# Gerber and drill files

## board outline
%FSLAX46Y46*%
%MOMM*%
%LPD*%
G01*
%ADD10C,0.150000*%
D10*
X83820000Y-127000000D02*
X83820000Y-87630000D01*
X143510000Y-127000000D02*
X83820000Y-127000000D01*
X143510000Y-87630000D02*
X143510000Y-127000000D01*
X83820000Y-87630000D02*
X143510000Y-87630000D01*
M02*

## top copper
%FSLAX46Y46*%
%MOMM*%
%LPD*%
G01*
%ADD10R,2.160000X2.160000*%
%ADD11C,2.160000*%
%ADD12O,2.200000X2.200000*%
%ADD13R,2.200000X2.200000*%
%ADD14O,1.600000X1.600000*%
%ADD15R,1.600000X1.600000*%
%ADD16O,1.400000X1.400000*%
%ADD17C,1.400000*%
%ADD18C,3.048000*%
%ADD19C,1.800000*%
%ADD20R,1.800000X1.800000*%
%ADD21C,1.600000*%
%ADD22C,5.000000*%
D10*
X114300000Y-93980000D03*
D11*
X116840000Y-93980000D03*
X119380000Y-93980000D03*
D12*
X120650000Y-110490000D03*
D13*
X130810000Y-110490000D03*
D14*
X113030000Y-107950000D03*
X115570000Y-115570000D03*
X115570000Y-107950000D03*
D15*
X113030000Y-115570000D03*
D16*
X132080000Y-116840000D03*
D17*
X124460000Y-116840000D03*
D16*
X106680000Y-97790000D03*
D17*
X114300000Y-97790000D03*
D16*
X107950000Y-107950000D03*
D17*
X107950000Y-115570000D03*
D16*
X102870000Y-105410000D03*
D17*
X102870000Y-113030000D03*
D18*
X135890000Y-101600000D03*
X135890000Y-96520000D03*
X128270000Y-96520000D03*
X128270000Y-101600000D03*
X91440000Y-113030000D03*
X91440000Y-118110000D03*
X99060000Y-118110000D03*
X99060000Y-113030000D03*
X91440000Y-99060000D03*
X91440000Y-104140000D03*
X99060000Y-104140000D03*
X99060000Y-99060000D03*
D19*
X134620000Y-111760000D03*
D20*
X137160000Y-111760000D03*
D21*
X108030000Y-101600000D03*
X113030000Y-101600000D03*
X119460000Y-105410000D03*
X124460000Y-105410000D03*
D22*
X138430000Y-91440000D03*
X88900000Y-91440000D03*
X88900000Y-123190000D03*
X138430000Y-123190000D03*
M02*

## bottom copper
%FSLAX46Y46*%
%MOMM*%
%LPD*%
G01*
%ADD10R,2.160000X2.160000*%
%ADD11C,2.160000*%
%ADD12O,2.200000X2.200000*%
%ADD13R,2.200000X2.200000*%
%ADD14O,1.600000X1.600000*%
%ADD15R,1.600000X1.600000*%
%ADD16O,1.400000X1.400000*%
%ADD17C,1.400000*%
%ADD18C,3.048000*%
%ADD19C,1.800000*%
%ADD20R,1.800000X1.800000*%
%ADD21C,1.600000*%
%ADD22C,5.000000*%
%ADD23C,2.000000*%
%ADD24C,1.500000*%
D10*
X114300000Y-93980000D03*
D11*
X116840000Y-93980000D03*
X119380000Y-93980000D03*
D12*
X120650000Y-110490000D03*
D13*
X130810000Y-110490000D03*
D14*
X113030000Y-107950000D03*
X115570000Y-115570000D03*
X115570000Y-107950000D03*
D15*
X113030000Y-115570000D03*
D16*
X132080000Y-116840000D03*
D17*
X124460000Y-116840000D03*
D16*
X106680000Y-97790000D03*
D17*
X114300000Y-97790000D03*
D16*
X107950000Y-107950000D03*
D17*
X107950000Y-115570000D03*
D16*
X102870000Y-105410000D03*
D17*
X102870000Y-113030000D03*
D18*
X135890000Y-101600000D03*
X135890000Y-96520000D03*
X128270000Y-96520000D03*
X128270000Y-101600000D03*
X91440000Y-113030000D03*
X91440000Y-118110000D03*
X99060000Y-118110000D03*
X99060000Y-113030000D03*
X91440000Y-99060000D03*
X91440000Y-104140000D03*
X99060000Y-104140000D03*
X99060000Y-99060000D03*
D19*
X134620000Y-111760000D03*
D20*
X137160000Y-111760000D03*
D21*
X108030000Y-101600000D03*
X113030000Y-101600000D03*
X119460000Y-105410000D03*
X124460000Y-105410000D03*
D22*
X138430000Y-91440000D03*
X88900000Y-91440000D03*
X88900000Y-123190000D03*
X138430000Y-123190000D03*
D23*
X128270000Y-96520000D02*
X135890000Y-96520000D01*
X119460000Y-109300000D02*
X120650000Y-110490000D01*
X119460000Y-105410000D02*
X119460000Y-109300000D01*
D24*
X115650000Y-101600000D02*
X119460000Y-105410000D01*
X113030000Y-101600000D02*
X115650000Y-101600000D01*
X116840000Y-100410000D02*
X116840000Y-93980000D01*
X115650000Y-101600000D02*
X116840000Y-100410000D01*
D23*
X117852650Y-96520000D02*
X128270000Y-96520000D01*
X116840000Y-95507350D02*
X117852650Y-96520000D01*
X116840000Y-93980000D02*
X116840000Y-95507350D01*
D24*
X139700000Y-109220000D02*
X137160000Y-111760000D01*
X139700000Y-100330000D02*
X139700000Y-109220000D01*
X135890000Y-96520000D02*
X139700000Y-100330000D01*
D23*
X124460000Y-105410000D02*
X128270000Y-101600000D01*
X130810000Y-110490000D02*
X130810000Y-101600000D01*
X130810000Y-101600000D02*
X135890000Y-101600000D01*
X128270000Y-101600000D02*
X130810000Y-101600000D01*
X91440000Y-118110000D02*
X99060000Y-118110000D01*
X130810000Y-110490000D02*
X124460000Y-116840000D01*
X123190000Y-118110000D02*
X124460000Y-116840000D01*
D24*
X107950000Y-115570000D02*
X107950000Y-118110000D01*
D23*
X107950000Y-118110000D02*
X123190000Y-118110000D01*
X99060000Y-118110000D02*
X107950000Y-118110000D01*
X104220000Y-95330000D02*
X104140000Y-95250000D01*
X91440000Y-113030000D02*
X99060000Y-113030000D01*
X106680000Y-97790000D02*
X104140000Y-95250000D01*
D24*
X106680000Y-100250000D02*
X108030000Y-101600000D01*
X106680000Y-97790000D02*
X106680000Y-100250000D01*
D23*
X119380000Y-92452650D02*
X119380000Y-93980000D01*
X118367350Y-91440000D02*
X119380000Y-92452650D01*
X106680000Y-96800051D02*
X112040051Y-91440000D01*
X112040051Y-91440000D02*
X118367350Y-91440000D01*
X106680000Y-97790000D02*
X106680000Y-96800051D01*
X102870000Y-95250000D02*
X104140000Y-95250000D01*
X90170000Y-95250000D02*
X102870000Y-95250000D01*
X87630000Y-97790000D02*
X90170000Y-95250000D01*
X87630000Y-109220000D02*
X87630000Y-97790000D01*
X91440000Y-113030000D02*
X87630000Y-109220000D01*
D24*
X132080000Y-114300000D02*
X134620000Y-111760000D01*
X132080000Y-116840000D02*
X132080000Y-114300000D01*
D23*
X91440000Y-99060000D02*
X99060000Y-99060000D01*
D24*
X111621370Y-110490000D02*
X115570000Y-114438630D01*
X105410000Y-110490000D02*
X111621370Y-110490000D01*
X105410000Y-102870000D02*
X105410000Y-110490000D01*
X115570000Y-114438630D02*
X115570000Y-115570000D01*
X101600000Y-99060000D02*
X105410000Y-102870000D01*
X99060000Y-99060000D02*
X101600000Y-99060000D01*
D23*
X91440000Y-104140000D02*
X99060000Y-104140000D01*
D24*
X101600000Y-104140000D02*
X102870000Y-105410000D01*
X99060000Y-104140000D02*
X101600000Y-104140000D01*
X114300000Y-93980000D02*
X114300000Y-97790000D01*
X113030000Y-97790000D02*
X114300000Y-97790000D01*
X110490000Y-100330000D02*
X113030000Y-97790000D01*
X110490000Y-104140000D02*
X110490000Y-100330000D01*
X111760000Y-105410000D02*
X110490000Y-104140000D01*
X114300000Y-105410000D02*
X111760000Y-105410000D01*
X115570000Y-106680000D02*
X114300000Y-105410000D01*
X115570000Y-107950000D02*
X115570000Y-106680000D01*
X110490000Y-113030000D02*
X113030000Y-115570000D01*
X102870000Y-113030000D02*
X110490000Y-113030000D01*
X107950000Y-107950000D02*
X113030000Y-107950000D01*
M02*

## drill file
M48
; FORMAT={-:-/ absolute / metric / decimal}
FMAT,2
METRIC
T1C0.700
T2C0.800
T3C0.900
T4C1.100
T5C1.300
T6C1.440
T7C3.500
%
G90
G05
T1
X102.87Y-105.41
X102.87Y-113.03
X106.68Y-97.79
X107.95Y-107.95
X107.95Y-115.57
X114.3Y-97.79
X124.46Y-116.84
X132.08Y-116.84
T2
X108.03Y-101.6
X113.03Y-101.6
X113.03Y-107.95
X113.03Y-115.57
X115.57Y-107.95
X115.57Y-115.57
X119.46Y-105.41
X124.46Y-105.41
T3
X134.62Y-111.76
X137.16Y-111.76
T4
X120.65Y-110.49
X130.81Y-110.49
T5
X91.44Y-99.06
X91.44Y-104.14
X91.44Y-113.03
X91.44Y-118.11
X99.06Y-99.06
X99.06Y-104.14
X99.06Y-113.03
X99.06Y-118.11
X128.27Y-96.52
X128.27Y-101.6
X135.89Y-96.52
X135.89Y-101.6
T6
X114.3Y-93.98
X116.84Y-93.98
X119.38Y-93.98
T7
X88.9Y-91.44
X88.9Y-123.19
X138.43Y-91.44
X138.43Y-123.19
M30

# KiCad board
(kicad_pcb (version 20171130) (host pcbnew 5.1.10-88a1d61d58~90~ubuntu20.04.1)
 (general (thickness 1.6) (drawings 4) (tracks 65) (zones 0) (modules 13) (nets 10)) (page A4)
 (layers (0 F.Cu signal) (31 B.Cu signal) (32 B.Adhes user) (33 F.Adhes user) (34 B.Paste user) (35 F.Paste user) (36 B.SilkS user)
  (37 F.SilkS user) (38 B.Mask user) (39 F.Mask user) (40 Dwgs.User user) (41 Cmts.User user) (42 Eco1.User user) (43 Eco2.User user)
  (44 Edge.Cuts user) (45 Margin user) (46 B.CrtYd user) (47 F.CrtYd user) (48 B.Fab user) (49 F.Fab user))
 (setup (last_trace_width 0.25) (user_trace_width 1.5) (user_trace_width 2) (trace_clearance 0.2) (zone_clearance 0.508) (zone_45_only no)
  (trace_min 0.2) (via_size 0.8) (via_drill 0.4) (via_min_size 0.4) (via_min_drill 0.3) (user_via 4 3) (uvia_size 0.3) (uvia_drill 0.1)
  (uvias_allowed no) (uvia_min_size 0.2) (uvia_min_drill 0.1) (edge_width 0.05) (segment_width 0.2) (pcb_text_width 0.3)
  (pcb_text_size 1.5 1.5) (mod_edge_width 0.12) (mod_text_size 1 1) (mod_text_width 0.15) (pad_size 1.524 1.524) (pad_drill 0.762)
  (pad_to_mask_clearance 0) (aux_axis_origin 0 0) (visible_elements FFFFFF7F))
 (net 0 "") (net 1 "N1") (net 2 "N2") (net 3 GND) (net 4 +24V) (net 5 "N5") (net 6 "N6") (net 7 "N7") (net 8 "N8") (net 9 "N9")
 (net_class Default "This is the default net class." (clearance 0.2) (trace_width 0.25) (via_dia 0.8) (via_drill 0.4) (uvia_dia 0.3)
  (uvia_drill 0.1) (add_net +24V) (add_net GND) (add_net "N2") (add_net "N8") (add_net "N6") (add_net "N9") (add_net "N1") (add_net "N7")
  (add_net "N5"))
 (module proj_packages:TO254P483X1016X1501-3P (layer F.Cu) (at 114.3 93.98)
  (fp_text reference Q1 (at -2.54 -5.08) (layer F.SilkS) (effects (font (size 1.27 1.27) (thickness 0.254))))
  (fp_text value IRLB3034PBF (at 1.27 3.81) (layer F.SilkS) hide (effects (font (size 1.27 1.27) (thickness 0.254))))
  (pad 1 thru_hole rect (at 0 0) (size 2.16 2.16) (drill 1.44) (layers *.Cu *.Mask) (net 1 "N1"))
  (pad 2 thru_hole circle (at 2.54 0) (size 2.16 2.16) (drill 1.44) (layers *.Cu *.Mask) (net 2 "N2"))
  (pad 3 thru_hole circle (at 5.08 0) (size 2.16 2.16) (drill 1.44) (layers *.Cu *.Mask) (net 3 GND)))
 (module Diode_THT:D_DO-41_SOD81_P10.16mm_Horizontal (layer F.Cu) (at 130.81 110.49 180)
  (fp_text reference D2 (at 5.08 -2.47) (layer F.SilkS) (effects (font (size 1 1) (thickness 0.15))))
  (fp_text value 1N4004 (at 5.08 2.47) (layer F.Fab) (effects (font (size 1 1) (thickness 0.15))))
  (pad 2 thru_hole oval (at 10.16 0 180) (size 2.2 2.2) (drill 1.1) (layers *.Cu *.Mask) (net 2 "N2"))
  (pad 1 thru_hole rect (at 0 0 180) (size 2.2 2.2) (drill 1.1) (layers *.Cu *.Mask) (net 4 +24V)))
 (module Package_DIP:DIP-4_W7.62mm (layer F.Cu) (at 113.03 115.57 90)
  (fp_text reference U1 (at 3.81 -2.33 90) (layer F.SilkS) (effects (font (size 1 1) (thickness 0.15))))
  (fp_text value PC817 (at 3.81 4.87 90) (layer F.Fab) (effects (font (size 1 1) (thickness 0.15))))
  (pad 4 thru_hole oval (at 7.62 0 90) (size 1.6 1.6) (drill 0.8) (layers *.Cu *.Mask) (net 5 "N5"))
  (pad 2 thru_hole oval (at 0 2.54 90) (size 1.6 1.6) (drill 0.8) (layers *.Cu *.Mask) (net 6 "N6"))
  (pad 3 thru_hole oval (at 7.62 2.54 90) (size 1.6 1.6) (drill 0.8) (layers *.Cu *.Mask) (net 1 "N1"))
  (pad 1 thru_hole rect (at 0 0 90) (size 1.6 1.6) (drill 0.8) (layers *.Cu *.Mask) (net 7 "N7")))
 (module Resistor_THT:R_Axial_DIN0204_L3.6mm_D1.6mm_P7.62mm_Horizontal (layer F.Cu) (at 124.46 116.84)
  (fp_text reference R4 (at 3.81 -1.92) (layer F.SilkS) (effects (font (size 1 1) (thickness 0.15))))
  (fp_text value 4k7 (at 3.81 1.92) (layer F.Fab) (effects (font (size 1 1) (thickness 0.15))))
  (pad 2 thru_hole oval (at 7.62 0) (size 1.4 1.4) (drill 0.7) (layers *.Cu *.Mask) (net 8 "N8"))
  (pad 1 thru_hole circle (at 0 0) (size 1.4 1.4) (drill 0.7) (layers *.Cu *.Mask) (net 4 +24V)))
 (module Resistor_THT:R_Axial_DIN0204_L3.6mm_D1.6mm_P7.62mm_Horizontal (layer F.Cu) (at 114.3 97.79 180)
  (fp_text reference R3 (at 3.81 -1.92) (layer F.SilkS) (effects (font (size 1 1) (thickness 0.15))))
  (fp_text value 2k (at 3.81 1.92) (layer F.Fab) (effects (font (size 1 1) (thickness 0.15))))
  (pad 2 thru_hole oval (at 7.62 0 180) (size 1.4 1.4) (drill 0.7) (layers *.Cu *.Mask) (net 3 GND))
  (pad 1 thru_hole circle (at 0 0 180) (size 1.4 1.4) (drill 0.7) (layers *.Cu *.Mask) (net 1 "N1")))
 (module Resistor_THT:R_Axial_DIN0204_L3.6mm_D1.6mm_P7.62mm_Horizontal (layer F.Cu) (at 107.95 115.57 90)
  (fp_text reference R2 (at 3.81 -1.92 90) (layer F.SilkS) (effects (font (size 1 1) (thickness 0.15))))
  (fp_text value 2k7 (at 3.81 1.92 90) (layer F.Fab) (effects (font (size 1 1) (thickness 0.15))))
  (pad 2 thru_hole oval (at 7.62 0 90) (size 1.4 1.4) (drill 0.7) (layers *.Cu *.Mask) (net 5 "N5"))
  (pad 1 thru_hole circle (at 0 0 90) (size 1.4 1.4) (drill 0.7) (layers *.Cu *.Mask) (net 4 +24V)))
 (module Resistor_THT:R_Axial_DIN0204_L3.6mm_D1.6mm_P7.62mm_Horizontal (layer F.Cu) (at 102.87 113.03 90)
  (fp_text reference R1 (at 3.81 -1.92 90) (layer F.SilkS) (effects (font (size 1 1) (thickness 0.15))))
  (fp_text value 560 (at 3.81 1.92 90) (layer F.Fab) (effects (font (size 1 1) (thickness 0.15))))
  (pad 2 thru_hole oval (at 7.62 0 90) (size 1.4 1.4) (drill 0.7) (layers *.Cu *.Mask) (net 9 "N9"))
  (pad 1 thru_hole circle (at 0 0 90) (size 1.4 1.4) (drill 0.7) (layers *.Cu *.Mask) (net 7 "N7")))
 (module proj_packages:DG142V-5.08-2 (layer F.Cu) (at 135.89 99.06 90)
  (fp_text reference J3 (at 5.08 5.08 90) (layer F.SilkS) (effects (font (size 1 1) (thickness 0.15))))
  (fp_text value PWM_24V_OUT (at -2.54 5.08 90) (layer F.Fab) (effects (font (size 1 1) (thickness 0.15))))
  (pad 1 thru_hole circle (at -2.54 0 90) (size 3.048 3.048) (drill 1.3) (layers *.Cu *.Mask) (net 4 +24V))
  (pad 2 thru_hole circle (at 2.54 0 90) (size 3.048 3.048) (drill 1.3) (layers *.Cu *.Mask) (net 2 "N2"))
  (pad 2 thru_hole circle (at 2.54 -7.62 90) (size 3.048 3.048) (drill 1.3) (layers *.Cu *.Mask) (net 2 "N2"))
  (pad 1 thru_hole circle (at -2.54 -7.62 90) (size 3.048 3.048) (drill 1.3) (layers *.Cu *.Mask) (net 4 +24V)))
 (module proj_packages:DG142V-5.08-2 (layer F.Cu) (at 91.44 115.57 270)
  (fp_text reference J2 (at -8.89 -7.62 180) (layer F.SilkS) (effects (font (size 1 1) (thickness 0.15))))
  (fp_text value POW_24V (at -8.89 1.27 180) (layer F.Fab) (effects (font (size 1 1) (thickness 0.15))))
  (pad 1 thru_hole circle (at -2.54 0 270) (size 3.048 3.048) (drill 1.3) (layers *.Cu *.Mask) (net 3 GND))
  (pad 2 thru_hole circle (at 2.54 0 270) (size 3.048 3.048) (drill 1.3) (layers *.Cu *.Mask) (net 4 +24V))
  (pad 2 thru_hole circle (at 2.54 -7.62 270) (size 3.048 3.048) (drill 1.3) (layers *.Cu *.Mask) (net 4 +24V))
  (pad 1 thru_hole circle (at -2.54 -7.62 270) (size 3.048 3.048) (drill 1.3) (layers *.Cu *.Mask) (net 3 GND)))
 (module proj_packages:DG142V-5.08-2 (layer F.Cu) (at 91.44 101.6 270)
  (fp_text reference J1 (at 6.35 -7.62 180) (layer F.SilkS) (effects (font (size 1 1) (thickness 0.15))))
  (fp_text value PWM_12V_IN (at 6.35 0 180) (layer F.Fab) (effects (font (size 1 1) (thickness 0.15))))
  (pad 1 thru_hole circle (at -2.54 0 270) (size 3.048 3.048) (drill 1.3) (layers *.Cu *.Mask) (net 6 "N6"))
  (pad 2 thru_hole circle (at 2.54 0 270) (size 3.048 3.048) (drill 1.3) (layers *.Cu *.Mask) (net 9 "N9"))
  (pad 2 thru_hole circle (at 2.54 -7.62 270) (size 3.048 3.048) (drill 1.3) (layers *.Cu *.Mask) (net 9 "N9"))
  (pad 1 thru_hole circle (at -2.54 -7.62 270) (size 3.048 3.048) (drill 1.3) (layers *.Cu *.Mask) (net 6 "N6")))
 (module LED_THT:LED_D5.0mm (layer F.Cu) (at 137.16 111.76 180)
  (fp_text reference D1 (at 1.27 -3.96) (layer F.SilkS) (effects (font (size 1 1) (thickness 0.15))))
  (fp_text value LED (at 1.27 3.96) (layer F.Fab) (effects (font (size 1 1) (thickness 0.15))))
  (pad 2 thru_hole circle (at 2.54 0 180) (size 1.8 1.8) (drill 0.9) (layers *.Cu *.Mask) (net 8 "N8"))
  (pad 1 thru_hole rect (at 0 0 180) (size 1.8 1.8) (drill 0.9) (layers *.Cu *.Mask) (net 2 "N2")))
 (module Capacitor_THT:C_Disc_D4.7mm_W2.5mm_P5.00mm (layer F.Cu) (at 113.03 101.6 180)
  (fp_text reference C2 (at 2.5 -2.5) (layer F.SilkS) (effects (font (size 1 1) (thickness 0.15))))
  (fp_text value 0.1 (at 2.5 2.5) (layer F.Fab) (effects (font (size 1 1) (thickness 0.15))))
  (pad 2 thru_hole circle (at 5 0 180) (size 1.6 1.6) (drill 0.8) (layers *.Cu *.Mask) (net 3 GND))
  (pad 1 thru_hole circle (at 0 0 180) (size 1.6 1.6) (drill 0.8) (layers *.Cu *.Mask) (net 2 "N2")))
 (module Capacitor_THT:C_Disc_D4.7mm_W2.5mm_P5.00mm (layer F.Cu) (at 124.46 105.41 180)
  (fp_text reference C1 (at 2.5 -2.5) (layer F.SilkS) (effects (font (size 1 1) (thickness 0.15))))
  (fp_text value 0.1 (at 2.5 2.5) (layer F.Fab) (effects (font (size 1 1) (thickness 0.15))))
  (pad 2 thru_hole circle (at 5 0 180) (size 1.6 1.6) (drill 0.8) (layers *.Cu *.Mask) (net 2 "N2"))
  (pad 1 thru_hole circle (at 0 0 180) (size 1.6 1.6) (drill 0.8) (layers *.Cu *.Mask) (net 4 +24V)))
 (gr_line (start 83.82 127) (end 83.82 87.63) (layer Edge.Cuts) (width 0.15))
 (gr_line (start 143.51 127) (end 83.82 127) (layer Edge.Cuts) (width 0.15))
 (gr_line (start 143.51 87.63) (end 143.51 127) (layer Edge.Cuts) (width 0.15))
 (gr_line (start 83.82 87.63) (end 143.51 87.63) (layer Edge.Cuts) (width 0.15))
 (via (at 138.43 91.44) (size 5) (drill 3.5) (layers F.Cu B.Cu) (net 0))
 (via (at 88.9 91.44) (size 5) (drill 3.5) (layers F.Cu B.Cu) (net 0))
 (via (at 88.9 123.19) (size 5) (drill 3.5) (layers F.Cu B.Cu) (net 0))
 (via (at 138.43 123.19) (size 5) (drill 3.5) (layers F.Cu B.Cu) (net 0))
 (segment (start 128.27 96.52) (end 135.89 96.52) (width 2) (layer B.Cu) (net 2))
 (segment (start 119.46 109.3) (end 120.65 110.49) (width 2) (layer B.Cu) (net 2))
 (segment (start 119.46 105.41) (end 119.46 109.3) (width 2) (layer B.Cu) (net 2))
 (segment (start 115.65 101.6) (end 119.46 105.41) (width 1.5) (layer B.Cu) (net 2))
 (segment (start 113.03 101.6) (end 115.65 101.6) (width 1.5) (layer B.Cu) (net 2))
 (segment (start 116.84 100.41) (end 116.84 93.98) (width 1.5) (layer B.Cu) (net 2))
 (segment (start 115.65 101.6) (end 116.84 100.41) (width 1.5) (layer B.Cu) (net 2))
 (segment (start 117.85265 96.52) (end 128.27 96.52) (width 2) (layer B.Cu) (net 2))
 (segment (start 116.84 95.50735) (end 117.85265 96.52) (width 2) (layer B.Cu) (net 2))
 (segment (start 116.84 93.98) (end 116.84 95.50735) (width 2) (layer B.Cu) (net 2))
 (segment (start 139.7 109.22) (end 137.16 111.76) (width 1.5) (layer B.Cu) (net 2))
 (segment (start 139.7 100.33) (end 139.7 109.22) (width 1.5) (layer B.Cu) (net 2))
 (segment (start 135.89 96.52) (end 139.7 100.33) (width 1.5) (layer B.Cu) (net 2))
 (segment (start 124.46 105.41) (end 128.27 101.6) (width 2) (layer B.Cu) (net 4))
 (segment (start 130.81 110.49) (end 130.81 101.6) (width 2) (layer B.Cu) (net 4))
 (segment (start 130.81 101.6) (end 135.89 101.6) (width 2) (layer B.Cu) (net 4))
 (segment (start 128.27 101.6) (end 130.81 101.6) (width 2) (layer B.Cu) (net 4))
 (segment (start 91.44 118.11) (end 99.06 118.11) (width 2) (layer B.Cu) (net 4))
 (segment (start 130.81 110.49) (end 124.46 116.84) (width 2) (layer B.Cu) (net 4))
 (segment (start 123.19 118.11) (end 124.46 116.84) (width 2) (layer B.Cu) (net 4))
 (segment (start 107.95 115.57) (end 107.95 118.11) (width 1.5) (layer B.Cu) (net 4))
 (segment (start 107.95 118.11) (end 123.19 118.11) (width 2) (layer B.Cu) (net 4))
 (segment (start 99.06 118.11) (end 107.95 118.11) (width 2) (layer B.Cu) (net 4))
 (segment (start 104.22 95.33) (end 104.14 95.25) (width 2) (layer B.Cu) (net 3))
 (segment (start 91.44 113.03) (end 99.06 113.03) (width 2) (layer B.Cu) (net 3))
 (segment (start 106.68 97.79) (end 104.14 95.25) (width 2) (layer B.Cu) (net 3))
 (segment (start 106.68 100.25) (end 108.03 101.6) (width 1.5) (layer B.Cu) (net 3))
 (segment (start 106.68 97.79) (end 106.68 100.25) (width 1.5) (layer B.Cu) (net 3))
 (segment (start 119.38 92.45265) (end 119.38 93.98) (width 2) (layer B.Cu) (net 3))
 (segment (start 118.36735 91.44) (end 119.38 92.45265) (width 2) (layer B.Cu) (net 3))
 (segment (start 106.68 96.800051) (end 112.040051 91.44) (width 2) (layer B.Cu) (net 3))
 (segment (start 112.040051 91.44) (end 118.36735 91.44) (width 2) (layer B.Cu) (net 3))
 (segment (start 106.68 97.79) (end 106.68 96.800051) (width 2) (layer B.Cu) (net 3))
 (segment (start 102.87 95.25) (end 104.14 95.25) (width 2) (layer B.Cu) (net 3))
 (segment (start 90.17 95.25) (end 102.87 95.25) (width 2) (layer B.Cu) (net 3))
 (segment (start 87.63 97.79) (end 90.17 95.25) (width 2) (layer B.Cu) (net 3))
 (segment (start 87.63 109.22) (end 87.63 97.79) (width 2) (layer B.Cu) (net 3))
 (segment (start 91.44 113.03) (end 87.63 109.22) (width 2) (layer B.Cu) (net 3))
 (segment (start 132.08 114.3) (end 134.62 111.76) (width 1.5) (layer B.Cu) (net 8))
 (segment (start 132.08 116.84) (end 132.08 114.3) (width 1.5) (layer B.Cu) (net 8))
 (segment (start 91.44 99.06) (end 99.06 99.06) (width 2) (layer B.Cu) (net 6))
 (segment (start 111.62137 110.49) (end 115.57 114.43863) (width 1.5) (layer B.Cu) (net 6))
 (segment (start 105.41 110.49) (end 111.62137 110.49) (width 1.5) (layer B.Cu) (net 6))
 (segment (start 105.41 102.87) (end 105.41 110.49) (width 1.5) (layer B.Cu) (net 6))
 (segment (start 115.57 114.43863) (end 115.57 115.57) (width 1.5) (layer B.Cu) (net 6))
 (segment (start 101.6 99.06) (end 105.41 102.87) (width 1.5) (layer B.Cu) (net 6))
 (segment (start 99.06 99.06) (end 101.6 99.06) (width 1.5) (layer B.Cu) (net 6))
 (segment (start 91.44 104.14) (end 99.06 104.14) (width 2) (layer B.Cu) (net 9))
 (segment (start 101.6 104.14) (end 102.87 105.41) (width 1.5) (layer B.Cu) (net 9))
 (segment (start 99.06 104.14) (end 101.6 104.14) (width 1.5) (layer B.Cu) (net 9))
 (segment (start 114.3 93.98) (end 114.3 97.79) (width 1.5) (layer B.Cu) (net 1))
 (segment (start 113.03 97.79) (end 114.3 97.79) (width 1.5) (layer B.Cu) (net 1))
 (segment (start 110.49 100.33) (end 113.03 97.79) (width 1.5) (layer B.Cu) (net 1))
 (segment (start 110.49 104.14) (end 110.49 100.33) (width 1.5) (layer B.Cu) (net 1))
 (segment (start 111.76 105.41) (end 110.49 104.14) (width 1.5) (layer B.Cu) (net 1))
 (segment (start 114.3 105.41) (end 111.76 105.41) (width 1.5) (layer B.Cu) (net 1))
 (segment (start 115.57 106.68) (end 114.3 105.41) (width 1.5) (layer B.Cu) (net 1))
 (segment (start 115.57 107.95) (end 115.57 106.68) (width 1.5) (layer B.Cu) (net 1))
 (segment (start 110.49 113.03) (end 113.03 115.57) (width 1.5) (layer B.Cu) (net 7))
 (segment (start 102.87 113.03) (end 110.49 113.03) (width 1.5) (layer B.Cu) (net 7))
 (segment (start 107.95 107.95) (end 113.03 107.95) (width 1.5) (layer B.Cu) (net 5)))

